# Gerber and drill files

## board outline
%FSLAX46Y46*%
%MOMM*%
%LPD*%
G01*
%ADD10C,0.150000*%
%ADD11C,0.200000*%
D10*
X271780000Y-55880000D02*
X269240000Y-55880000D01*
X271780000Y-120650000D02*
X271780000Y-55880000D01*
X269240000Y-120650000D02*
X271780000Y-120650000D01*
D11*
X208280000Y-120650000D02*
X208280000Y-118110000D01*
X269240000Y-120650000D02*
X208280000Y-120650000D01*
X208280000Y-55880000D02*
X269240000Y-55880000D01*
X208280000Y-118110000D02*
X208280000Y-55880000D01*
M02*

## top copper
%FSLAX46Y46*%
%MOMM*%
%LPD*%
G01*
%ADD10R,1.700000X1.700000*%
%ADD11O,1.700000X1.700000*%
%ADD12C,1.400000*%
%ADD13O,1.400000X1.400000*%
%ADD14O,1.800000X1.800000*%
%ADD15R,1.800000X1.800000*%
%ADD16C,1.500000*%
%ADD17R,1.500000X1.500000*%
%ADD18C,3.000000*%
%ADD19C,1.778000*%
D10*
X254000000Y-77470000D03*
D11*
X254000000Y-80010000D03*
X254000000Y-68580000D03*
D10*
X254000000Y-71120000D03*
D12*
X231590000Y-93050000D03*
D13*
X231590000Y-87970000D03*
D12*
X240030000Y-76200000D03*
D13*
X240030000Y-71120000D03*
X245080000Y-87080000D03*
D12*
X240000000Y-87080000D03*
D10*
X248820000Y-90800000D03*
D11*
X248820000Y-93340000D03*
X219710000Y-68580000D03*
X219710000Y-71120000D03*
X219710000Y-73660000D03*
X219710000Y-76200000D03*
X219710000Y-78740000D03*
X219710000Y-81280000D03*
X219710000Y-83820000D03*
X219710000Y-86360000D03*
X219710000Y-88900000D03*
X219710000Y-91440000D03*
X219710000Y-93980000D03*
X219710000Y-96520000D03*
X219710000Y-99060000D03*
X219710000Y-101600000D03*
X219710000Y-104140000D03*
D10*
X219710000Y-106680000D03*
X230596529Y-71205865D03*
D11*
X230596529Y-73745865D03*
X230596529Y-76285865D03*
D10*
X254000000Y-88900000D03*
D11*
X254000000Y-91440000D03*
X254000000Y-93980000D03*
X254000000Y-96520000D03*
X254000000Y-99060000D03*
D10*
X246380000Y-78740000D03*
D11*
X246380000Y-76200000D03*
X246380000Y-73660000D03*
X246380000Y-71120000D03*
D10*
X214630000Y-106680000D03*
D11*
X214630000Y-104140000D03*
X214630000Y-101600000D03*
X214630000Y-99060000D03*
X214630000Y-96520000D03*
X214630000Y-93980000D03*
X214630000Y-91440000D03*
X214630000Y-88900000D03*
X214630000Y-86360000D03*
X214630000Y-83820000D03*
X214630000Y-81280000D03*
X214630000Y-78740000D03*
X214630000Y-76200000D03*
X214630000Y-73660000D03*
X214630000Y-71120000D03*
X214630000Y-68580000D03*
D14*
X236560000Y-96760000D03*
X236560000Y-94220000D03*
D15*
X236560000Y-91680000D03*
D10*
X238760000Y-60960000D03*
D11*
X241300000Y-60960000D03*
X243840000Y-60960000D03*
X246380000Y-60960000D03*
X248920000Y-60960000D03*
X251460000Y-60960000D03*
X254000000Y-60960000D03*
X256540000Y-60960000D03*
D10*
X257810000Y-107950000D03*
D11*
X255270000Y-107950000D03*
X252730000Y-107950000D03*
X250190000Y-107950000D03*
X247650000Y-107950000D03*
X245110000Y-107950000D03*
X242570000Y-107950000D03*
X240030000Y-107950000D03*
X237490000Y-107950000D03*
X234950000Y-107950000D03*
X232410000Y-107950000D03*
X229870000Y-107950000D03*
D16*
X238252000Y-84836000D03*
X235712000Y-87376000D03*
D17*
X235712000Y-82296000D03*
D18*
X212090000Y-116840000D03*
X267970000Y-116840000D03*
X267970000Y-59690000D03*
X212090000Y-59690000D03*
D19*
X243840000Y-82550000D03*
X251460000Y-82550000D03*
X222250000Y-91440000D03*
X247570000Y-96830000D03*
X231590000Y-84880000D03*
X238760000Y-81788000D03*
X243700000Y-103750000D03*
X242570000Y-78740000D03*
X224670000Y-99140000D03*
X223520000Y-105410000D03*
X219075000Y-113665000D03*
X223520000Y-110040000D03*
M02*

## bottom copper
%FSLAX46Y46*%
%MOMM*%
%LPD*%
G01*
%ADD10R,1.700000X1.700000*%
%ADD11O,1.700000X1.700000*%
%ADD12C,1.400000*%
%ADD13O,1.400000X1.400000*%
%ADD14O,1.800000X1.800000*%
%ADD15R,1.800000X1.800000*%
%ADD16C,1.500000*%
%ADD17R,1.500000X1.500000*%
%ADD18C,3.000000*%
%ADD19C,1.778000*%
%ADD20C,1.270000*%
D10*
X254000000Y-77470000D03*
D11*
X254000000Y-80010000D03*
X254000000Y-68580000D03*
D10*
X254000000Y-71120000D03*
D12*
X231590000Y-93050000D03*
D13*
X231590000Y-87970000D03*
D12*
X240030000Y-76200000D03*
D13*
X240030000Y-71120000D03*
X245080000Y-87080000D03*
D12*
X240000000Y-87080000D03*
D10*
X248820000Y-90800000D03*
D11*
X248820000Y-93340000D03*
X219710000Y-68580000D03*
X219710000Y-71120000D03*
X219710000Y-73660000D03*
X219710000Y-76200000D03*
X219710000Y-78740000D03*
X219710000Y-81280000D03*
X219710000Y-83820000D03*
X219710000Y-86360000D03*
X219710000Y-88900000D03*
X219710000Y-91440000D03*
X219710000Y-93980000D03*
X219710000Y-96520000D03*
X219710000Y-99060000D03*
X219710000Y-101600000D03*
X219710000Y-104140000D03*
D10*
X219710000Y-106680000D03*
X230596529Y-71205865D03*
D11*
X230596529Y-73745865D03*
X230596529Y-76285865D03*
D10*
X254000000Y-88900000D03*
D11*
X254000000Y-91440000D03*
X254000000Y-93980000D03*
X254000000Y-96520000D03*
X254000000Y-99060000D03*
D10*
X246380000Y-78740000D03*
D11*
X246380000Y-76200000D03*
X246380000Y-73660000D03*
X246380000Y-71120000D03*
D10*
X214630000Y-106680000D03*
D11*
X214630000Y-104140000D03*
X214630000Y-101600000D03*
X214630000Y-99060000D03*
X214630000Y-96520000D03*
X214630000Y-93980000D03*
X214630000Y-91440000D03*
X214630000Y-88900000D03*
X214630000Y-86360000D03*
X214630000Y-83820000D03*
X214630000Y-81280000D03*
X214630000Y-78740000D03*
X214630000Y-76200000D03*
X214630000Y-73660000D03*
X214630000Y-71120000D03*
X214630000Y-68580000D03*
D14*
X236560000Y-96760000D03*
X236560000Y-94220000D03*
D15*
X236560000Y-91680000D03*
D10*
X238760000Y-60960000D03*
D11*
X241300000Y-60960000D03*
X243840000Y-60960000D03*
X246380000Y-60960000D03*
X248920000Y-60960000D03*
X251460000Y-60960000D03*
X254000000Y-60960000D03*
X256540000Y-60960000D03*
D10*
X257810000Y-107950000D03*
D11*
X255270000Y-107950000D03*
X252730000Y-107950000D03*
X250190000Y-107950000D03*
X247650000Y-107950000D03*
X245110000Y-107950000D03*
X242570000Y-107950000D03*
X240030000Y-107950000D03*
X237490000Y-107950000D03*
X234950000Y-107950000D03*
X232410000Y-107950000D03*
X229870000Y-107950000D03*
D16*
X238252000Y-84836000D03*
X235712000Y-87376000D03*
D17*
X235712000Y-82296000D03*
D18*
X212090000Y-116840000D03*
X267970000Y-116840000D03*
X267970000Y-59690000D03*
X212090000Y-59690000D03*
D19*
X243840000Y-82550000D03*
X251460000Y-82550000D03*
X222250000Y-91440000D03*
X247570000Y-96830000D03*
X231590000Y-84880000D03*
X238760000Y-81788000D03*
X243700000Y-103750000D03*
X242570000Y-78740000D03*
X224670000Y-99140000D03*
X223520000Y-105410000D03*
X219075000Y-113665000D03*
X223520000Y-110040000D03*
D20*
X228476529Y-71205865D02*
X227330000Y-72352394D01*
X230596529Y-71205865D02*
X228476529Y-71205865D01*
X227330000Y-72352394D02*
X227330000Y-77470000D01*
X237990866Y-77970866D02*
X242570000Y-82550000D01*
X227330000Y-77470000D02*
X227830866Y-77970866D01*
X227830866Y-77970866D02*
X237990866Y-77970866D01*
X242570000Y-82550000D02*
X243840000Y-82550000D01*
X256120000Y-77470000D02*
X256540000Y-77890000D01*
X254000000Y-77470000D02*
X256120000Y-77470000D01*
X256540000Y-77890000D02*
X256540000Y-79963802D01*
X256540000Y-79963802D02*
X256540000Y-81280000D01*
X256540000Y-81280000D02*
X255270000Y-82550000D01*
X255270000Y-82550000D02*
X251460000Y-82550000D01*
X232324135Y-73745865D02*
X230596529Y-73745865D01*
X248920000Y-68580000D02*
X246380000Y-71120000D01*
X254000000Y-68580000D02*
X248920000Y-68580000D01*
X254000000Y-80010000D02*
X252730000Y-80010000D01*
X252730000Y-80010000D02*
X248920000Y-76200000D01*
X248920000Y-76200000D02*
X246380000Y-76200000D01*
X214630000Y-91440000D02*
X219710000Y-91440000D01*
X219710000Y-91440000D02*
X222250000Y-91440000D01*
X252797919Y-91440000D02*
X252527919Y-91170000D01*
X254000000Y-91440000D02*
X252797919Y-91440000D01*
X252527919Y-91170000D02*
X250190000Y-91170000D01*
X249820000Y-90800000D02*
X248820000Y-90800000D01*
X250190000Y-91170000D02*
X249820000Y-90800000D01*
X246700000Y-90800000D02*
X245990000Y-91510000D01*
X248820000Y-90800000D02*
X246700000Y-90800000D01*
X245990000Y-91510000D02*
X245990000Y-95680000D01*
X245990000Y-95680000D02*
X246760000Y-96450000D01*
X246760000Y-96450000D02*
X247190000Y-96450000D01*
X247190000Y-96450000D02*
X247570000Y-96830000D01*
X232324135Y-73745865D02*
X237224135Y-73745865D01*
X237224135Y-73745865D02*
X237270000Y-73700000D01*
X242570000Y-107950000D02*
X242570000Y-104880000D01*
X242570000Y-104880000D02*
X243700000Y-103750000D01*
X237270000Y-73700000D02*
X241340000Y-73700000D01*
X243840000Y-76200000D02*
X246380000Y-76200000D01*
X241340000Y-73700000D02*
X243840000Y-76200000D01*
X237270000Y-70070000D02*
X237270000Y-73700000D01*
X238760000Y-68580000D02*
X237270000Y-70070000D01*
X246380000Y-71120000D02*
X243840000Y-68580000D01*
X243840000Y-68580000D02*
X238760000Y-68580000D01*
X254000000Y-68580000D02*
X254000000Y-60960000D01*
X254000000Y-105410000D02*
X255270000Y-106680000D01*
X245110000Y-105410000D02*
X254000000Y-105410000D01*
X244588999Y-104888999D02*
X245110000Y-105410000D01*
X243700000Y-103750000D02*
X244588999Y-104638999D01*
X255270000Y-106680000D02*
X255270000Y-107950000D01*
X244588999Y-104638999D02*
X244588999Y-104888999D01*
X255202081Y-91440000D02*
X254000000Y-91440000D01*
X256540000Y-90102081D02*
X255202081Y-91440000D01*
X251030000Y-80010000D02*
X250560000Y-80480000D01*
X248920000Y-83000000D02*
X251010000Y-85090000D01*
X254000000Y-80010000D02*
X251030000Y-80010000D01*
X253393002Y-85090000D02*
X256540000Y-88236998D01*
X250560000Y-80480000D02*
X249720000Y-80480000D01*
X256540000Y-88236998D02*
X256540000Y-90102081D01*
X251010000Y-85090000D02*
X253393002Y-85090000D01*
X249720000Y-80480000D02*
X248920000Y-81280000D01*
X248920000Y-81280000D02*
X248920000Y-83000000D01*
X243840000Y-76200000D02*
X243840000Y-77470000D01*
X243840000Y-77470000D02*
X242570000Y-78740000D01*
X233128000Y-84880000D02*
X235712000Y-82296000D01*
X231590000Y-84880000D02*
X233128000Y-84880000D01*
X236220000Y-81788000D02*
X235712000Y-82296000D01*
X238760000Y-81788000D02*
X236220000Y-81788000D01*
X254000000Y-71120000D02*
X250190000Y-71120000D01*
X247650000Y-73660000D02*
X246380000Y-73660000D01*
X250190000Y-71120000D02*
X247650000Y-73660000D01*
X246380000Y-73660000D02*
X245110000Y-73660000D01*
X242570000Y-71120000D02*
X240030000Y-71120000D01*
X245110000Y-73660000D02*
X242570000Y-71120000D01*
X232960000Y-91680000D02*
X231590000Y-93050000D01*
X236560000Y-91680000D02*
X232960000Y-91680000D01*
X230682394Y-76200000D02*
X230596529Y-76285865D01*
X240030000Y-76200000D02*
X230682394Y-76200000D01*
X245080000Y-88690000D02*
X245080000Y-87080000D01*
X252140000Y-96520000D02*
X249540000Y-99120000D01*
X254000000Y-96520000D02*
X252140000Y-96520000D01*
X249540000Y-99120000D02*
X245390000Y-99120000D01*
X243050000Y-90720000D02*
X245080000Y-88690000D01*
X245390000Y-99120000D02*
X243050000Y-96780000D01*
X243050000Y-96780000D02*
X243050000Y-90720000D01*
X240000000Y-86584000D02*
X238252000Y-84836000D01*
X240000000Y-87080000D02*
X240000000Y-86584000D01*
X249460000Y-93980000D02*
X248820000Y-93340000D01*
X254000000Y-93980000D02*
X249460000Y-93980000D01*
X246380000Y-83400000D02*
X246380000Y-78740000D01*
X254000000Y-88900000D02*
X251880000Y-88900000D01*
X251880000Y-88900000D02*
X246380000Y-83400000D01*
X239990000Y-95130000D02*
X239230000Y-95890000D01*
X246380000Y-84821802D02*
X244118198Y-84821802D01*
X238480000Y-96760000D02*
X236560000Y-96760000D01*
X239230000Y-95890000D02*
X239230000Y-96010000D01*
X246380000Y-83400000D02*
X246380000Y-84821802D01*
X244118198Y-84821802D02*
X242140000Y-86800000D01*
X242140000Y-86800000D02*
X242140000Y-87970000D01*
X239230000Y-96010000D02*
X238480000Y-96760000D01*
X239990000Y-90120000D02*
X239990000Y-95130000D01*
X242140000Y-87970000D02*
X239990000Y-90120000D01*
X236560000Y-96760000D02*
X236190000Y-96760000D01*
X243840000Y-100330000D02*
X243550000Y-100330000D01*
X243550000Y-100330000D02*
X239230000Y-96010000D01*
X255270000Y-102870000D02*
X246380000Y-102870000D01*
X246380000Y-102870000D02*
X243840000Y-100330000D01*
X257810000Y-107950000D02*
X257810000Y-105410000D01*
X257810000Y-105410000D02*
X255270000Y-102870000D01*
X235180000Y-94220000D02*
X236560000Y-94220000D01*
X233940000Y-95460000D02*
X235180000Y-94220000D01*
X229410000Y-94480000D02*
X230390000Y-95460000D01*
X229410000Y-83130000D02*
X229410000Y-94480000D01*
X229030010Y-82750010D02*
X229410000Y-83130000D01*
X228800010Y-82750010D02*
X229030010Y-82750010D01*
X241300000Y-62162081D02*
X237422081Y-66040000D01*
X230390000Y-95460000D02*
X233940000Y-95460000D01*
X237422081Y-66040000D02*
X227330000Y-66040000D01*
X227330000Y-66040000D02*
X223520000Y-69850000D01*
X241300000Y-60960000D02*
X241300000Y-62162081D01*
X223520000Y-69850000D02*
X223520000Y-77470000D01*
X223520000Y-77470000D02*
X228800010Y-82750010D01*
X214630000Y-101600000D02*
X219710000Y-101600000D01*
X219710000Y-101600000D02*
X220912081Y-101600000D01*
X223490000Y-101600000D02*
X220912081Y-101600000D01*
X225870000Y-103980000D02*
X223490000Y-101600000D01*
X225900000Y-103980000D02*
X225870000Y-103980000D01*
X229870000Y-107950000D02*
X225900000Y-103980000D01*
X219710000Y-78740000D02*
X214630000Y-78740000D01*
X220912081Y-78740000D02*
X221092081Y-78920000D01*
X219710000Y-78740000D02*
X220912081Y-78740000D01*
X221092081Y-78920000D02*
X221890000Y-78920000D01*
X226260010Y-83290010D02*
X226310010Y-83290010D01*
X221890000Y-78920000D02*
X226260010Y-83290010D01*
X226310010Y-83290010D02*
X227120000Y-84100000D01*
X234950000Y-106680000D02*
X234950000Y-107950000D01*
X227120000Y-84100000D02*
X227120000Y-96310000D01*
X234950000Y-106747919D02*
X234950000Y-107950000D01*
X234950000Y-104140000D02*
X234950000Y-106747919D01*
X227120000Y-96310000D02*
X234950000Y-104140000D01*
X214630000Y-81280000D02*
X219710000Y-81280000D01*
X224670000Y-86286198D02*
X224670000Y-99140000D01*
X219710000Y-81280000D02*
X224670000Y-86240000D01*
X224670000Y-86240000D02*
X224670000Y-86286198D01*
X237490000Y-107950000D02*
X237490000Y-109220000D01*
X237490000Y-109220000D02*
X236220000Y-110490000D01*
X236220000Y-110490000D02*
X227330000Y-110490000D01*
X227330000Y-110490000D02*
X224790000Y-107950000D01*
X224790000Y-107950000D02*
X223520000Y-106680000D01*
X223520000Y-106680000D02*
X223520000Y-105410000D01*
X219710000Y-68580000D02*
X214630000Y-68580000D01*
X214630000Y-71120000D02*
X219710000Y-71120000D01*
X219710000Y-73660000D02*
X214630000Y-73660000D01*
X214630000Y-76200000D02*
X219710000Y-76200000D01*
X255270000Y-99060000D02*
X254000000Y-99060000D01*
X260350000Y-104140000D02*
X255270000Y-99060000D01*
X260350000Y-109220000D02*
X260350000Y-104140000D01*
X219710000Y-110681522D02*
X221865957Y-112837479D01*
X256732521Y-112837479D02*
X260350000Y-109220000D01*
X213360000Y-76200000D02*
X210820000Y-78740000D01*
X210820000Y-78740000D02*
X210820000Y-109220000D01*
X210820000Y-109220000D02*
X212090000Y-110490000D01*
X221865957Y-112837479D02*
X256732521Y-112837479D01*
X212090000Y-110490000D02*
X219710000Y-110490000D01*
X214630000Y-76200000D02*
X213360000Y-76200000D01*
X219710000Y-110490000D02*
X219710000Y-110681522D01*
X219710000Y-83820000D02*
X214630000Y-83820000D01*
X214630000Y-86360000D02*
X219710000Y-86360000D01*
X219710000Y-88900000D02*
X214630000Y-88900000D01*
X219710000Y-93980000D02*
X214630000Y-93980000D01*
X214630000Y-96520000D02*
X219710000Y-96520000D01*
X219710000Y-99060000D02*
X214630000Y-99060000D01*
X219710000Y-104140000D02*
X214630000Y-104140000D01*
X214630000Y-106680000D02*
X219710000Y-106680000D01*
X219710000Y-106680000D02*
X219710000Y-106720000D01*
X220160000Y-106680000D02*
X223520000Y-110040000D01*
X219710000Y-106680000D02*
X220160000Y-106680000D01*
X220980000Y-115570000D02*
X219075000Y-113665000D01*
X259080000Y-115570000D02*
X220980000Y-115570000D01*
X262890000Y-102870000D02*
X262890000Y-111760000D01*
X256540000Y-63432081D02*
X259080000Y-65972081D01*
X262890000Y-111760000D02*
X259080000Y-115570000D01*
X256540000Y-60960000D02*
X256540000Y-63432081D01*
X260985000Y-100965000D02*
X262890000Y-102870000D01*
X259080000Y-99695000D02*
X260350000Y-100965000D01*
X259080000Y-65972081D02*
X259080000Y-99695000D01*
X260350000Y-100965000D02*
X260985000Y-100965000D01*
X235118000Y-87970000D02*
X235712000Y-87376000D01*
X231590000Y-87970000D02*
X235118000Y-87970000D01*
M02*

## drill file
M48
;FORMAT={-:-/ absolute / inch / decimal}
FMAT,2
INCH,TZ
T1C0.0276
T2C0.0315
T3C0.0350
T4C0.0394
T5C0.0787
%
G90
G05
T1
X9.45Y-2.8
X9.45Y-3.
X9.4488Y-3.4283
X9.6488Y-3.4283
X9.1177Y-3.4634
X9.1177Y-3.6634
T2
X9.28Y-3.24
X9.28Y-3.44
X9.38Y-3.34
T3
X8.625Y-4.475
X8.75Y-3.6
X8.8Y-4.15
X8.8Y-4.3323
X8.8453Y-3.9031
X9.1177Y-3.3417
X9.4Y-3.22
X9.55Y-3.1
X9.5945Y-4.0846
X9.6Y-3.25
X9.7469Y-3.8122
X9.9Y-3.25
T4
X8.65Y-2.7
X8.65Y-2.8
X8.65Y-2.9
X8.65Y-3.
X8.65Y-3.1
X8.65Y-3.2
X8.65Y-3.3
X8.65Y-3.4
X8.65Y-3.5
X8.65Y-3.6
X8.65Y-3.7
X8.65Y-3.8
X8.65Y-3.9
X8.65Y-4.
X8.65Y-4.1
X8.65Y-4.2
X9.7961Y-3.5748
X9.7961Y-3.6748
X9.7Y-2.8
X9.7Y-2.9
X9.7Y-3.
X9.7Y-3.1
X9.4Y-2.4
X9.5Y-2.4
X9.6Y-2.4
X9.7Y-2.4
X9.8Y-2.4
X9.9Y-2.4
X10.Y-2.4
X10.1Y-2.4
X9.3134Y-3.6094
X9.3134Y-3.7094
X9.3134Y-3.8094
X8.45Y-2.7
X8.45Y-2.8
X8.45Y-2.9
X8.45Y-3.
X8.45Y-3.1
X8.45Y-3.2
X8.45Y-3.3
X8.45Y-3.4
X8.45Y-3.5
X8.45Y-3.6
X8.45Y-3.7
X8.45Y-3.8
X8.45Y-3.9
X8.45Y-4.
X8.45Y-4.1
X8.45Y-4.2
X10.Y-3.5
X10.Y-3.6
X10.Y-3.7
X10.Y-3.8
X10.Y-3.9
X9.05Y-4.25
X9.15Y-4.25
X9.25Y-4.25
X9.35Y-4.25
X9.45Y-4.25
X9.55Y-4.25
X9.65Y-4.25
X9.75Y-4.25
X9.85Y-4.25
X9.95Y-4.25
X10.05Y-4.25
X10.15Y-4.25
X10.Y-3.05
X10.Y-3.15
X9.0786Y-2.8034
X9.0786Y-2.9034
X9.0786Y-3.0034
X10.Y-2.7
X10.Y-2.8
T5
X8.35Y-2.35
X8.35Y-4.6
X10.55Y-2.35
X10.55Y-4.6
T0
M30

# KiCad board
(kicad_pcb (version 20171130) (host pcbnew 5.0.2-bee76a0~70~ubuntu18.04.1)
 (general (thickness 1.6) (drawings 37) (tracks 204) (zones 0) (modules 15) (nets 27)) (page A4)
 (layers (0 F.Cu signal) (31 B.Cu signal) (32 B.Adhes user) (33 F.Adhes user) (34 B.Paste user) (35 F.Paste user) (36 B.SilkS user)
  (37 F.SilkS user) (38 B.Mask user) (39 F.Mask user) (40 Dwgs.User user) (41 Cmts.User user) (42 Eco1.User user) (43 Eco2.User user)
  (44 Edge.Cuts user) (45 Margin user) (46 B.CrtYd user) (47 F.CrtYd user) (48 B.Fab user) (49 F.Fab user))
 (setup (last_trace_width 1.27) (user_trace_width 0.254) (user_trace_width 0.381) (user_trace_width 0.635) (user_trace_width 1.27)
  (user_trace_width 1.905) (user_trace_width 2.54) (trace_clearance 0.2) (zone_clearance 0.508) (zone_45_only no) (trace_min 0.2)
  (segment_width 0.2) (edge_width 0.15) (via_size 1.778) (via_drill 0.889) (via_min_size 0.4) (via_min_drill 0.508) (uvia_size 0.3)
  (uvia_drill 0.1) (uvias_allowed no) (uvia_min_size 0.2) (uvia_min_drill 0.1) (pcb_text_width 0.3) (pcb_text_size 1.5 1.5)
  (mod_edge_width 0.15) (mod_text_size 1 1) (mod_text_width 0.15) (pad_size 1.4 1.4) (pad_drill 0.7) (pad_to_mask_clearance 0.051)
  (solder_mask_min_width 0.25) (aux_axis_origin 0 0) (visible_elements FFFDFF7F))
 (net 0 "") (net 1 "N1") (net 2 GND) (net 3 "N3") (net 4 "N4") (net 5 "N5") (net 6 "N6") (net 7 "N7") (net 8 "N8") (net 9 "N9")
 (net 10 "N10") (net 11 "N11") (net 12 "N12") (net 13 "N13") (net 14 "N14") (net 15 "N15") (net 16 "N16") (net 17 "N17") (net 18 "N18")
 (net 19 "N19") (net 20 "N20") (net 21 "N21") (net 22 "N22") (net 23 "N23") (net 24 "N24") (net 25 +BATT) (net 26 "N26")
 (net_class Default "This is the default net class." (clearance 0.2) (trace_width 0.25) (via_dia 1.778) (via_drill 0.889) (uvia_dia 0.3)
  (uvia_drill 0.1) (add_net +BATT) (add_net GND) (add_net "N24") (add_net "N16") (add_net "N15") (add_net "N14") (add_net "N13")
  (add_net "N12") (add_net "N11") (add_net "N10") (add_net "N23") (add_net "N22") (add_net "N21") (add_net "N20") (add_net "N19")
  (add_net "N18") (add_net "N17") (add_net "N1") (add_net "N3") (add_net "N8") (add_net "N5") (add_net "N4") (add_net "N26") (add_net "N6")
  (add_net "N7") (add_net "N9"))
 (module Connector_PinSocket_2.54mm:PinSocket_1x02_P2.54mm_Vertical (layer F.Cu) (at 254 77.47)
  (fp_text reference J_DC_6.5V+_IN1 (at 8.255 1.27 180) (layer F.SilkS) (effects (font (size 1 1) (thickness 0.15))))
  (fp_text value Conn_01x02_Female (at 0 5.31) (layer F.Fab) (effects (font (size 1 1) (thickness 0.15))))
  (pad 1 thru_hole rect (at 0 0) (size 1.7 1.7) (drill 1) (layers *.Cu *.Mask) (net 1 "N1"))
  (pad 2 thru_hole oval (at 0 2.54) (size 1.7 1.7) (drill 1) (layers *.Cu *.Mask) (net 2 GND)))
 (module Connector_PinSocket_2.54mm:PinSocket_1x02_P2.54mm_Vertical (layer F.Cu) (at 254 71.12 180)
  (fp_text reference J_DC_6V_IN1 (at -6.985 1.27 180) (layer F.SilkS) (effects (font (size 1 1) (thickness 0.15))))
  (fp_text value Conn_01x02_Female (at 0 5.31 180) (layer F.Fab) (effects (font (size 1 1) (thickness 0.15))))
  (pad 2 thru_hole oval (at 0 2.54 180) (size 1.7 1.7) (drill 1) (layers *.Cu *.Mask) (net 2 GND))
  (pad 1 thru_hole rect (at 0 0 180) (size 1.7 1.7) (drill 1) (layers *.Cu *.Mask) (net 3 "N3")))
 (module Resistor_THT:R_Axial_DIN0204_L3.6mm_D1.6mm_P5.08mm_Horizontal (layer F.Cu) (at 231.59 93.05 90)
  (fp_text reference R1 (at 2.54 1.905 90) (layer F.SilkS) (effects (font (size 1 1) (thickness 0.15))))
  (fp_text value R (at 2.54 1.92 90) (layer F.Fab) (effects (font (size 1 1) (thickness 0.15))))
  (pad 1 thru_hole circle (at 0 0 90) (size 1.4 1.4) (drill 0.7) (layers *.Cu *.Mask) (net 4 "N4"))
  (pad 2 thru_hole oval (at 5.08 0 90) (size 1.4 1.4) (drill 0.7) (layers *.Cu *.Mask) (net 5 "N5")))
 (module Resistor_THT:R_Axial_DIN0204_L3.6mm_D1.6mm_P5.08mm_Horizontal (layer F.Cu) (at 240.03 76.2 90)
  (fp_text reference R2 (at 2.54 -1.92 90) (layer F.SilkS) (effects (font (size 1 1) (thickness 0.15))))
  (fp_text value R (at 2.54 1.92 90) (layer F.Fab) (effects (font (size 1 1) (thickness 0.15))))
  (pad 1 thru_hole circle (at 0 0 90) (size 1.4 1.4) (drill 0.7) (layers *.Cu *.Mask) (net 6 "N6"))
  (pad 2 thru_hole oval (at 5.08 0 90) (size 1.4 1.4) (drill 0.7) (layers *.Cu *.Mask) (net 3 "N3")))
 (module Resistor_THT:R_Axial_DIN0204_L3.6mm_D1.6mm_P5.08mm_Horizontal (layer F.Cu) (at 240 87.08)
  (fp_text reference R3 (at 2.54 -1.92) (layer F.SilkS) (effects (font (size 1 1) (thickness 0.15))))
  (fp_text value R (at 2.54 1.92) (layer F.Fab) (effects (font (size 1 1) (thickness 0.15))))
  (pad 2 thru_hole oval (at 5.08 0) (size 1.4 1.4) (drill 0.7) (layers *.Cu *.Mask) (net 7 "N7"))
  (pad 1 thru_hole circle (at 0 0) (size 1.4 1.4) (drill 0.7) (layers *.Cu *.Mask) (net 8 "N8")))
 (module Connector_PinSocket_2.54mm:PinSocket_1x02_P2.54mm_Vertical (layer F.Cu) (at 248.82 90.8)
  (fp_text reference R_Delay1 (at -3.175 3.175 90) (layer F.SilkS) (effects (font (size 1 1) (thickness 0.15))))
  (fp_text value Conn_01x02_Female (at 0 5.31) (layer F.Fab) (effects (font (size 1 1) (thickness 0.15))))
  (pad 1 thru_hole rect (at 0 0) (size 1.7 1.7) (drill 1) (layers *.Cu *.Mask) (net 2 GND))
  (pad 2 thru_hole oval (at 0 2.54) (size 1.7 1.7) (drill 1) (layers *.Cu *.Mask) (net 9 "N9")))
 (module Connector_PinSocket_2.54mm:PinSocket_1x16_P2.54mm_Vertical (layer F.Cu) (at 219.71 106.68 180)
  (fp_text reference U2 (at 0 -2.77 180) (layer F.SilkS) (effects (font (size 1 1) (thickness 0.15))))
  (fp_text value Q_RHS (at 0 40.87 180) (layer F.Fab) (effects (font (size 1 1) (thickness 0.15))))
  (pad 16 thru_hole oval (at 0 38.1 180) (size 1.7 1.7) (drill 1) (layers *.Cu *.Mask) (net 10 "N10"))
  (pad 15 thru_hole oval (at 0 35.56 180) (size 1.7 1.7) (drill 1) (layers *.Cu *.Mask) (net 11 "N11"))
  (pad 14 thru_hole oval (at 0 33.02 180) (size 1.7 1.7) (drill 1) (layers *.Cu *.Mask) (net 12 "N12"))
  (pad 13 thru_hole oval (at 0 30.48 180) (size 1.7 1.7) (drill 1) (layers *.Cu *.Mask) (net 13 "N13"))
  (pad 12 thru_hole oval (at 0 27.94 180) (size 1.7 1.7) (drill 1) (layers *.Cu *.Mask) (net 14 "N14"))
  (pad 11 thru_hole oval (at 0 25.4 180) (size 1.7 1.7) (drill 1) (layers *.Cu *.Mask) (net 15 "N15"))
  (pad 10 thru_hole oval (at 0 22.86 180) (size 1.7 1.7) (drill 1) (layers *.Cu *.Mask) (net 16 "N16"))
  (pad 9 thru_hole oval (at 0 20.32 180) (size 1.7 1.7) (drill 1) (layers *.Cu *.Mask) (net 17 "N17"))
  (pad 8 thru_hole oval (at 0 17.78 180) (size 1.7 1.7) (drill 1) (layers *.Cu *.Mask) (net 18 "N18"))
  (pad 7 thru_hole oval (at 0 15.24 180) (size 1.7 1.7) (drill 1) (layers *.Cu *.Mask) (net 2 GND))
  (pad 6 thru_hole oval (at 0 12.7 180) (size 1.7 1.7) (drill 1) (layers *.Cu *.Mask) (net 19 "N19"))
  (pad 5 thru_hole oval (at 0 10.16 180) (size 1.7 1.7) (drill 1) (layers *.Cu *.Mask) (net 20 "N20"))
  (pad 4 thru_hole oval (at 0 7.62 180) (size 1.7 1.7) (drill 1) (layers *.Cu *.Mask) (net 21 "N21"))
  (pad 3 thru_hole oval (at 0 5.08 180) (size 1.7 1.7) (drill 1) (layers *.Cu *.Mask) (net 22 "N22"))
  (pad 2 thru_hole oval (at 0 2.54 180) (size 1.7 1.7) (drill 1) (layers *.Cu *.Mask) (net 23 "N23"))
  (pad 1 thru_hole rect (at 0 0 180) (size 1.7 1.7) (drill 1) (layers *.Cu *.Mask) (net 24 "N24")))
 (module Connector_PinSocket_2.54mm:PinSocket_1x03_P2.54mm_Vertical (layer F.Cu) (at 230.596529 71.205865)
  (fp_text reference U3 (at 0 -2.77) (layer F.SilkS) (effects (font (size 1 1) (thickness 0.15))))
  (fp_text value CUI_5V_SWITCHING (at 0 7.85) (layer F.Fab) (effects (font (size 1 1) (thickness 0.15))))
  (pad 1 thru_hole rect (at 0 0) (size 1.7 1.7) (drill 1) (layers *.Cu *.Mask) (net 1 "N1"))
  (pad 2 thru_hole oval (at 0 2.54) (size 1.7 1.7) (drill 1) (layers *.Cu *.Mask) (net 2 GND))
  (pad 3 thru_hole oval (at 0 5.08) (size 1.7 1.7) (drill 1) (layers *.Cu *.Mask) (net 6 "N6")))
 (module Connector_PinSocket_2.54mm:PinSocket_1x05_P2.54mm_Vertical (layer F.Cu) (at 254 88.9)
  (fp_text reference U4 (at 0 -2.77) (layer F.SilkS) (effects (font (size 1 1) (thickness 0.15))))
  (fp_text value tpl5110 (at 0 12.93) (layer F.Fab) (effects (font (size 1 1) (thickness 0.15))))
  (pad 1 thru_hole rect (at 0 0) (size 1.7 1.7) (drill 1) (layers *.Cu *.Mask) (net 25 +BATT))
  (pad 2 thru_hole oval (at 0 2.54) (size 1.7 1.7) (drill 1) (layers *.Cu *.Mask) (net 2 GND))
  (pad 3 thru_hole oval (at 0 5.08) (size 1.7 1.7) (drill 1) (layers *.Cu *.Mask) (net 9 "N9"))
  (pad 4 thru_hole oval (at 0 7.62) (size 1.7 1.7) (drill 1) (layers *.Cu *.Mask) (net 7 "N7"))
  (pad 5 thru_hole oval (at 0 10.16) (size 1.7 1.7) (drill 1) (layers *.Cu *.Mask) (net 13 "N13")))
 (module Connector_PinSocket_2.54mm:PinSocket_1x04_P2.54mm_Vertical (layer F.Cu) (at 246.38 78.74 180)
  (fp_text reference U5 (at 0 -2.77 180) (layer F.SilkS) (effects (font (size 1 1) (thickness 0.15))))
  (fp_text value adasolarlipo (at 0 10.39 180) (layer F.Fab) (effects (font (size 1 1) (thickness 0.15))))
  (pad 1 thru_hole rect (at 0 0 180) (size 1.7 1.7) (drill 1) (layers *.Cu *.Mask) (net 25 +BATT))
  (pad 2 thru_hole oval (at 0 2.54 180) (size 1.7 1.7) (drill 1) (layers *.Cu *.Mask) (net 2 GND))
  (pad 3 thru_hole oval (at 0 5.08 180) (size 1.7 1.7) (drill 1) (layers *.Cu *.Mask) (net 3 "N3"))
  (pad 4 thru_hole oval (at 0 7.62 180) (size 1.7 1.7) (drill 1) (layers *.Cu *.Mask) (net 2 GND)))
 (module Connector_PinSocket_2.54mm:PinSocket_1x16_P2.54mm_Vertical (layer F.Cu) (at 214.63 106.68 180)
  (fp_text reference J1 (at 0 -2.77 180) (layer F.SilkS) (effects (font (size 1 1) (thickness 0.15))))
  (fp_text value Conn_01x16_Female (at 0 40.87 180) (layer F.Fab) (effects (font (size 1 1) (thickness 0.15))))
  (pad 1 thru_hole rect (at 0 0 180) (size 1.7 1.7) (drill 1) (layers *.Cu *.Mask) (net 24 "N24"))
  (pad 2 thru_hole oval (at 0 2.54 180) (size 1.7 1.7) (drill 1) (layers *.Cu *.Mask) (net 23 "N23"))
  (pad 3 thru_hole oval (at 0 5.08 180) (size 1.7 1.7) (drill 1) (layers *.Cu *.Mask) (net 22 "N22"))
  (pad 4 thru_hole oval (at 0 7.62 180) (size 1.7 1.7) (drill 1) (layers *.Cu *.Mask) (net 21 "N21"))
  (pad 5 thru_hole oval (at 0 10.16 180) (size 1.7 1.7) (drill 1) (layers *.Cu *.Mask) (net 20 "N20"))
  (pad 6 thru_hole oval (at 0 12.7 180) (size 1.7 1.7) (drill 1) (layers *.Cu *.Mask) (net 19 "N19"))
  (pad 7 thru_hole oval (at 0 15.24 180) (size 1.7 1.7) (drill 1) (layers *.Cu *.Mask) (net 2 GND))
  (pad 8 thru_hole oval (at 0 17.78 180) (size 1.7 1.7) (drill 1) (layers *.Cu *.Mask) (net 18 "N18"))
  (pad 9 thru_hole oval (at 0 20.32 180) (size 1.7 1.7) (drill 1) (layers *.Cu *.Mask) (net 17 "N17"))
  (pad 10 thru_hole oval (at 0 22.86 180) (size 1.7 1.7) (drill 1) (layers *.Cu *.Mask) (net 16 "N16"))
  (pad 11 thru_hole oval (at 0 25.4 180) (size 1.7 1.7) (drill 1) (layers *.Cu *.Mask) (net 15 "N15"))
  (pad 12 thru_hole oval (at 0 27.94 180) (size 1.7 1.7) (drill 1) (layers *.Cu *.Mask) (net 14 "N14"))
  (pad 13 thru_hole oval (at 0 30.48 180) (size 1.7 1.7) (drill 1) (layers *.Cu *.Mask) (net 13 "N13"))
  (pad 14 thru_hole oval (at 0 33.02 180) (size 1.7 1.7) (drill 1) (layers *.Cu *.Mask) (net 12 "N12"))
  (pad 15 thru_hole oval (at 0 35.56 180) (size 1.7 1.7) (drill 1) (layers *.Cu *.Mask) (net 11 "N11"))
  (pad 16 thru_hole oval (at 0 38.1 180) (size 1.7 1.7) (drill 1) (layers *.Cu *.Mask) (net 10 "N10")))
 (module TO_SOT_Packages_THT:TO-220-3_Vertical (layer F.Cu) (at 236.56 91.68 270)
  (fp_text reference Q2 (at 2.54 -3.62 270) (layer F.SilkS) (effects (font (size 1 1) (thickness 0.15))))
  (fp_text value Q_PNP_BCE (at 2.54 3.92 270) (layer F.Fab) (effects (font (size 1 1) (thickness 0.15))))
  (pad 3 thru_hole oval (at 5.08 0 270) (size 1.8 1.8) (drill 1) (layers *.Cu *.Mask) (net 25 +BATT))
  (pad 2 thru_hole oval (at 2.54 0 270) (size 1.8 1.8) (drill 1) (layers *.Cu *.Mask) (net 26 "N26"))
  (pad 1 thru_hole rect (at 0 0 270) (size 1.8 1.8) (drill 1) (layers *.Cu *.Mask) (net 4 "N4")))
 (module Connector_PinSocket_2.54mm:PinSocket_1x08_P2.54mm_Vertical (layer F.Cu) (at 238.76 60.96 90)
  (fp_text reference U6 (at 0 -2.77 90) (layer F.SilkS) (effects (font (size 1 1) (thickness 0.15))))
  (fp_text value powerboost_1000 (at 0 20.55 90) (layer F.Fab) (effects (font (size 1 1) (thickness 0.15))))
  (pad 1 thru_hole rect (at 0 0 90) (size 1.7 1.7) (drill 1) (layers *.Cu *.Mask))
  (pad 2 thru_hole oval (at 0 2.54 90) (size 1.7 1.7) (drill 1) (layers *.Cu *.Mask) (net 26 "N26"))
  (pad 3 thru_hole oval (at 0 5.08 90) (size 1.7 1.7) (drill 1) (layers *.Cu *.Mask))
  (pad 4 thru_hole oval (at 0 7.62 90) (size 1.7 1.7) (drill 1) (layers *.Cu *.Mask))
  (pad 5 thru_hole oval (at 0 10.16 90) (size 1.7 1.7) (drill 1) (layers *.Cu *.Mask))
  (pad 6 thru_hole oval (at 0 12.7 90) (size 1.7 1.7) (drill 1) (layers *.Cu *.Mask))
  (pad 7 thru_hole oval (at 0 15.24 90) (size 1.7 1.7) (drill 1) (layers *.Cu *.Mask) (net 2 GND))
  (pad 8 thru_hole oval (at 0 17.78 90) (size 1.7 1.7) (drill 1) (layers *.Cu *.Mask) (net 24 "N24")))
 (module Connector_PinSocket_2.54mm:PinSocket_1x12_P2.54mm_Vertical (layer F.Cu) (at 257.81 107.95 270)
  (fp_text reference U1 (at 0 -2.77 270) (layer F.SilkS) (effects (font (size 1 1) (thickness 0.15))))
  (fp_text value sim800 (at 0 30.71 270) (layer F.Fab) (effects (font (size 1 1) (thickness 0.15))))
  (pad 1 thru_hole rect (at 0 0 270) (size 1.7 1.7) (drill 1) (layers *.Cu *.Mask) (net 25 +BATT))
  (pad 2 thru_hole oval (at 0 2.54 270) (size 1.7 1.7) (drill 1) (layers *.Cu *.Mask) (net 2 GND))
  (pad 3 thru_hole oval (at 0 5.08 270) (size 1.7 1.7) (drill 1) (layers *.Cu *.Mask))
  (pad 4 thru_hole oval (at 0 7.62 270) (size 1.7 1.7) (drill 1) (layers *.Cu *.Mask))
  (pad 5 thru_hole oval (at 0 10.16 270) (size 1.7 1.7) (drill 1) (layers *.Cu *.Mask))
  (pad 6 thru_hole oval (at 0 12.7 270) (size 1.7 1.7) (drill 1) (layers *.Cu *.Mask))
  (pad 7 thru_hole oval (at 0 15.24 270) (size 1.7 1.7) (drill 1) (layers *.Cu *.Mask) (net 2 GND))
  (pad 8 thru_hole oval (at 0 17.78 270) (size 1.7 1.7) (drill 1) (layers *.Cu *.Mask))
  (pad 9 thru_hole oval (at 0 20.32 270) (size 1.7 1.7) (drill 1) (layers *.Cu *.Mask) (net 15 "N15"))
  (pad 10 thru_hole oval (at 0 22.86 270) (size 1.7 1.7) (drill 1) (layers *.Cu *.Mask) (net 14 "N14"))
  (pad 11 thru_hole oval (at 0 25.4 270) (size 1.7 1.7) (drill 1) (layers *.Cu *.Mask))
  (pad 12 thru_hole oval (at 0 27.94 270) (size 1.7 1.7) (drill 1) (layers *.Cu *.Mask) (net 22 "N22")))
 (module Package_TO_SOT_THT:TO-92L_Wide (layer F.Cu) (at 235.712 82.296 270)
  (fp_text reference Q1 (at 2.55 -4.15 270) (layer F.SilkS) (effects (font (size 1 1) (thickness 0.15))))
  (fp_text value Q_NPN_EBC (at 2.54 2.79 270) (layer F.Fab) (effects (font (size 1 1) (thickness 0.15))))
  (pad 2 thru_hole circle (at 2.54 -2.54) (size 1.5 1.5) (drill 0.8) (layers *.Cu *.Mask) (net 8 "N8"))
  (pad 3 thru_hole circle (at 5.08 0) (size 1.5 1.5) (drill 0.8) (layers *.Cu *.Mask) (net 5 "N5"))
  (pad 1 thru_hole rect (at 0 0) (size 1.5 1.5) (drill 0.8) (layers *.Cu *.Mask) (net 2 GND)))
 (gr_line (start 271.78 55.88) (end 269.24 55.88) (layer Edge.Cuts) (width 0.15))
 (gr_line (start 271.78 120.65) (end 271.78 55.88) (layer Edge.Cuts) (width 0.15))
 (gr_line (start 269.24 120.65) (end 271.78 120.65) (layer Edge.Cuts) (width 0.15))
 (gr_line (start 208.28 120.65) (end 208.28 118.11) (layer Edge.Cuts) (width 0.2))
 (gr_line (start 269.24 120.65) (end 208.28 120.65) (layer Edge.Cuts) (width 0.2))
 (gr_line (start 208.28 55.88) (end 269.24 55.88) (layer Edge.Cuts) (width 0.2))
 (gr_line (start 208.28 118.11) (end 208.28 55.88) (layer Edge.Cuts) (width 0.2))
 (via (at 212.09 116.84) (size 3) (drill 2) (layers F.Cu B.Cu) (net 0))
 (via (at 267.97 116.84) (size 3) (drill 2) (layers F.Cu B.Cu) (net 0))
 (via (at 267.97 59.69) (size 3) (drill 2) (layers F.Cu B.Cu) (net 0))
 (via (at 212.09 59.69) (size 3) (drill 2) (layers F.Cu B.Cu) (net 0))
 (segment (start 228.476529 71.205865) (end 227.33 72.352394) (width 1.27) (layer B.Cu) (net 1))
 (segment (start 230.596529 71.205865) (end 228.476529 71.205865) (width 1.27) (layer B.Cu) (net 1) (status 10))
 (segment (start 227.33 72.352394) (end 227.33 77.47) (width 1.27) (layer B.Cu) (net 1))
 (segment (start 237.990866 77.970866) (end 242.57 82.55) (width 1.27) (layer B.Cu) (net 1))
 (segment (start 227.33 77.47) (end 227.830866 77.970866) (width 1.27) (layer B.Cu) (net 1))
 (segment (start 227.830866 77.970866) (end 237.990866 77.970866) (width 1.27) (layer B.Cu) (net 1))
 (via (at 243.84 82.55) (size 1.778) (drill 0.889) (layers F.Cu B.Cu) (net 1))
 (segment (start 242.57 82.55) (end 243.84 82.55) (width 1.27) (layer B.Cu) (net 1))
 (segment (start 256.12 77.47) (end 256.54 77.89) (width 1.27) (layer B.Cu) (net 1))
 (segment (start 254 77.47) (end 256.12 77.47) (width 1.27) (layer B.Cu) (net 1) (status 10))
 (segment (start 256.54 77.89) (end 256.54 79.963802) (width 1.27) (layer B.Cu) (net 1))
 (segment (start 256.54 79.963802) (end 256.54 81.28) (width 1.27) (layer B.Cu) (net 1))
 (segment (start 256.54 81.28) (end 255.27 82.55) (width 1.27) (layer B.Cu) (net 1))
 (via (at 251.46 82.55) (size 1.778) (drill 0.889) (layers F.Cu B.Cu) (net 1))
 (segment (start 255.27 82.55) (end 251.46 82.55) (width 1.27) (layer B.Cu) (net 1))
 (segment (start 232.324135 73.745865) (end 230.596529 73.745865) (width 1.27) (layer B.Cu) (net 2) (status 20))
 (segment (start 248.92 68.58) (end 246.38 71.12) (width 1.27) (layer B.Cu) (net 2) (status 20))
 (segment (start 254 68.58) (end 248.92 68.58) (width 1.27) (layer B.Cu) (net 2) (status 10))
 (segment (start 254 80.01) (end 252.73 80.01) (width 1.27) (layer B.Cu) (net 2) (status 10))
 (segment (start 252.73 80.01) (end 248.92 76.2) (width 1.27) (layer B.Cu) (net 2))
 (segment (start 248.92 76.2) (end 246.38 76.2) (width 1.27) (layer B.Cu) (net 2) (status 20))
 (segment (start 214.63 91.44) (end 219.71 91.44) (width 1.27) (layer B.Cu) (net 2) (status 30))
 (via (at 222.25 91.44) (size 1.778) (drill 0.889) (layers F.Cu B.Cu) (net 2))
 (segment (start 219.71 91.44) (end 222.25 91.44) (width 1.27) (layer B.Cu) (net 2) (status 10))
 (segment (start 252.797919 91.44) (end 252.527919 91.17) (width 1.27) (layer B.Cu) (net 2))
 (segment (start 254 91.44) (end 252.797919 91.44) (width 1.27) (layer B.Cu) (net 2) (status 10))
 (segment (start 252.527919 91.17) (end 250.19 91.17) (width 1.27) (layer B.Cu) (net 2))
 (segment (start 249.82 90.8) (end 248.82 90.8) (width 1.27) (layer B.Cu) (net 2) (status 20))
 (segment (start 250.19 91.17) (end 249.82 90.8) (width 1.27) (layer B.Cu) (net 2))
 (segment (start 246.7 90.8) (end 245.99 91.51) (width 1.27) (layer B.Cu) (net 2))
 (segment (start 248.82 90.8) (end 246.7 90.8) (width 1.27) (layer B.Cu) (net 2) (status 10))
 (segment (start 245.99 91.51) (end 245.99 95.68) (width 1.27) (layer B.Cu) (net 2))
 (segment (start 245.99 95.68) (end 246.76 96.45) (width 1.27) (layer B.Cu) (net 2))
 (via (at 247.57 96.83) (size 1.778) (drill 0.889) (layers F.Cu B.Cu) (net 2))
 (segment (start 246.76 96.45) (end 247.19 96.45) (width 1.27) (layer B.Cu) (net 2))
 (segment (start 247.19 96.45) (end 247.57 96.83) (width 1.27) (layer B.Cu) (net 2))
 (via (at 231.59 84.88) (size 1.778) (drill 0.889) (layers F.Cu B.Cu) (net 2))
 (via (at 238.76 81.788) (size 1.778) (drill 0.889) (layers F.Cu B.Cu) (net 2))
 (segment (start 232.324135 73.745865) (end 237.224135 73.745865) (width 1.27) (layer B.Cu) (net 2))
 (segment (start 237.224135 73.745865) (end 237.27 73.7) (width 1.27) (layer B.Cu) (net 2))
 (segment (start 254 71.12) (end 250.19 71.12) (width 1.27) (layer B.Cu) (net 3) (status 10))
 (segment (start 247.65 73.66) (end 246.38 73.66) (width 1.27) (layer B.Cu) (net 3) (status 20))
 (segment (start 250.19 71.12) (end 247.65 73.66) (width 1.27) (layer B.Cu) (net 3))
 (segment (start 232.96 91.68) (end 231.59 93.05) (width 1.27) (layer B.Cu) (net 4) (status 20))
 (segment (start 236.56 91.68) (end 232.96 91.68) (width 1.27) (layer B.Cu) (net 4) (status 10))
 (segment (start 230.682394 76.2) (end 230.596529 76.285865) (width 1.27) (layer B.Cu) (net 6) (status 30))
 (segment (start 240.03 76.2) (end 230.682394 76.2) (width 1.27) (layer B.Cu) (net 6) (status 30))
 (segment (start 245.08 88.69) (end 245.08 87.08) (width 1.27) (layer B.Cu) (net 7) (status 20))
 (segment (start 252.14 96.52) (end 249.54 99.12) (width 1.27) (layer B.Cu) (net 7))
 (segment (start 254 96.52) (end 252.14 96.52) (width 1.27) (layer B.Cu) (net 7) (status 10))
 (segment (start 249.54 99.12) (end 245.39 99.12) (width 1.27) (layer B.Cu) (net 7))
 (segment (start 243.05 90.72) (end 245.08 88.69) (width 1.27) (layer B.Cu) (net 7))
 (segment (start 245.39 99.12) (end 243.05 96.78) (width 1.27) (layer B.Cu) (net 7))
 (segment (start 243.05 96.78) (end 243.05 90.72) (width 1.27) (layer B.Cu) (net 7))
 (segment (start 249.46 93.98) (end 248.82 93.34) (width 1.27) (layer B.Cu) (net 9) (status 30))
 (segment (start 254 93.98) (end 249.46 93.98) (width 1.27) (layer B.Cu) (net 9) (status 30))
 (segment (start 246.38 83.4) (end 246.38 78.74) (width 1.27) (layer B.Cu) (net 25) (status 20))
 (segment (start 254 88.9) (end 251.88 88.9) (width 1.27) (layer B.Cu) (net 25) (status 10))
 (segment (start 251.88 88.9) (end 246.38 83.4) (width 1.27) (layer B.Cu) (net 25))
 (segment (start 239.99 95.13) (end 239.23 95.89) (width 1.27) (layer B.Cu) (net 25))
 (segment (start 246.38 84.821802) (end 244.118198 84.821802) (width 1.27) (layer B.Cu) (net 25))
 (segment (start 238.48 96.76) (end 236.56 96.76) (width 1.27) (layer B.Cu) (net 25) (status 20))
 (segment (start 239.23 95.89) (end 239.23 96.01) (width 1.27) (layer B.Cu) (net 25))
 (segment (start 246.38 83.4) (end 246.38 84.821802) (width 1.27) (layer B.Cu) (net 25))
 (segment (start 244.118198 84.821802) (end 242.14 86.8) (width 1.27) (layer B.Cu) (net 25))
 (segment (start 242.14 86.8) (end 242.14 87.97) (width 1.27) (layer B.Cu) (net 25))
 (segment (start 239.23 96.01) (end 238.48 96.76) (width 1.27) (layer B.Cu) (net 25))
 (segment (start 239.99 90.12) (end 239.99 95.13) (width 1.27) (layer B.Cu) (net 25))
 (segment (start 242.14 87.97) (end 239.99 90.12) (width 1.27) (layer B.Cu) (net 25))
 (segment (start 236.56 96.76) (end 236.19 96.76) (width 1.27) (layer B.Cu) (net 25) (status 30))
 (segment (start 214.63 101.6) (end 219.71 101.6) (width 1.27) (layer B.Cu) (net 22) (status 30))
 (segment (start 219.71 101.6) (end 220.912081 101.6) (width 1.27) (layer B.Cu) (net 22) (status 10))
 (segment (start 223.49 101.6) (end 220.912081 101.6) (width 1.27) (layer B.Cu) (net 22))
 (segment (start 225.87 103.98) (end 223.49 101.6) (width 1.27) (layer B.Cu) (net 22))
 (segment (start 219.71 78.74) (end 214.63 78.74) (width 1.27) (layer B.Cu) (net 14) (status 30))
 (via (at 243.7 103.75) (size 1.778) (drill 0.889) (layers F.Cu B.Cu) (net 2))
 (segment (start 242.57 107.95) (end 242.57 104.88) (width 1.27) (layer B.Cu) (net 2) (status 10))
 (segment (start 242.57 104.88) (end 243.7 103.75) (width 1.27) (layer B.Cu) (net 2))
 (segment (start 220.912081 78.74) (end 221.092081 78.92) (width 1.27) (layer B.Cu) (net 14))
 (segment (start 219.71 78.74) (end 220.912081 78.74) (width 1.27) (layer B.Cu) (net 14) (status 10))
 (segment (start 221.092081 78.92) (end 221.89 78.92) (width 1.27) (layer B.Cu) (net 14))
 (segment (start 226.26001 83.29001) (end 226.31001 83.29001) (width 1.27) (layer B.Cu) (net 14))
 (segment (start 221.89 78.92) (end 226.26001 83.29001) (width 1.27) (layer B.Cu) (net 14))
 (segment (start 226.31001 83.29001) (end 227.12 84.1) (width 1.27) (layer B.Cu) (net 14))
 (segment (start 214.63 81.28) (end 219.71 81.28) (width 1.27) (layer B.Cu) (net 15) (status 30))
 (segment (start 237.27 73.7) (end 241.34 73.7) (width 1.27) (layer B.Cu) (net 2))
 (segment (start 243.84 76.2) (end 246.38 76.2) (width 1.27) (layer B.Cu) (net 2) (status 20))
 (segment (start 241.34 73.7) (end 243.84 76.2) (width 1.27) (layer B.Cu) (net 2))
 (segment (start 237.27 70.07) (end 237.27 73.7) (width 1.27) (layer B.Cu) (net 2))
 (segment (start 238.76 68.58) (end 237.27 70.07) (width 1.27) (layer B.Cu) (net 2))
 (segment (start 246.38 71.12) (end 243.84 68.58) (width 1.27) (layer B.Cu) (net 2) (status 10))
 (segment (start 243.84 68.58) (end 238.76 68.58) (width 1.27) (layer B.Cu) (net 2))
 (segment (start 254 68.58) (end 254 60.96) (width 1.27) (layer B.Cu) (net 2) (status 30))
 (segment (start 254 105.41) (end 255.27 106.68) (width 1.27) (layer B.Cu) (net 2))
 (segment (start 245.11 105.41) (end 254 105.41) (width 1.27) (layer B.Cu) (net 2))
 (segment (start 244.588999 104.888999) (end 245.11 105.41) (width 1.27) (layer B.Cu) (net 2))
 (segment (start 243.7 103.75) (end 244.588999 104.638999) (width 1.27) (layer B.Cu) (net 2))
 (segment (start 255.27 106.68) (end 255.27 107.95) (width 1.27) (layer B.Cu) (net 2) (status 20))
 (segment (start 244.588999 104.638999) (end 244.588999 104.888999) (width 1.27) (layer B.Cu) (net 2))
 (segment (start 255.202081 91.44) (end 254 91.44) (width 1.27) (layer B.Cu) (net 2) (status 20))
 (segment (start 256.54 90.102081) (end 255.202081 91.44) (width 1.27) (layer B.Cu) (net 2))
 (segment (start 251.03 80.01) (end 250.56 80.48) (width 1.27) (layer B.Cu) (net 2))
 (segment (start 248.92 83) (end 251.01 85.09) (width 1.27) (layer B.Cu) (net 2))
 (segment (start 254 80.01) (end 251.03 80.01) (width 1.27) (layer B.Cu) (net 2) (status 10))
 (segment (start 253.393002 85.09) (end 256.54 88.236998) (width 1.27) (layer B.Cu) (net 2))
 (segment (start 250.56 80.48) (end 249.72 80.48) (width 1.27) (layer B.Cu) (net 2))
 (segment (start 256.54 88.236998) (end 256.54 90.102081) (width 1.27) (layer B.Cu) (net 2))
 (segment (start 251.01 85.09) (end 253.393002 85.09) (width 1.27) (layer B.Cu) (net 2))
 (segment (start 249.72 80.48) (end 248.92 81.28) (width 1.27) (layer B.Cu) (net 2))
 (segment (start 248.92 81.28) (end 248.92 83) (width 1.27) (layer B.Cu) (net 2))
 (via (at 242.57 78.74) (size 1.778) (drill 0.889) (layers F.Cu B.Cu) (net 2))
 (segment (start 243.84 76.2) (end 243.84 77.47) (width 1.27) (layer B.Cu) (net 2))
 (segment (start 243.84 77.47) (end 242.57 78.74) (width 1.27) (layer B.Cu) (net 2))
 (segment (start 233.128 84.88) (end 235.712 82.296) (width 1.27) (layer B.Cu) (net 2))
 (segment (start 231.59 84.88) (end 233.128 84.88) (width 1.27) (layer B.Cu) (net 2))
 (segment (start 236.22 81.788) (end 235.712 82.296) (width 1.27) (layer B.Cu) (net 2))
 (segment (start 238.76 81.788) (end 236.22 81.788) (width 1.27) (layer B.Cu) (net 2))
 (segment (start 246.38 73.66) (end 245.11 73.66) (width 1.27) (layer B.Cu) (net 3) (status 10))
 (segment (start 242.57 71.12) (end 240.03 71.12) (width 1.27) (layer B.Cu) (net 3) (status 20))
 (segment (start 245.11 73.66) (end 242.57 71.12) (width 1.27) (layer B.Cu) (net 3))
 (segment (start 240 86.584) (end 238.252 84.836) (width 1.27) (layer B.Cu) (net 8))
 (segment (start 240 87.08) (end 240 86.584) (width 1.27) (layer B.Cu) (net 8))
 (segment (start 243.84 100.33) (end 243.55 100.33) (width 1.27) (layer B.Cu) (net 25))
 (segment (start 243.55 100.33) (end 239.23 96.01) (width 1.27) (layer B.Cu) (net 25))
 (segment (start 255.27 102.87) (end 246.38 102.87) (width 1.27) (layer B.Cu) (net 25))
 (segment (start 246.38 102.87) (end 243.84 100.33) (width 1.27) (layer B.Cu) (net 25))
 (segment (start 257.81 107.95) (end 257.81 105.41) (width 1.27) (layer B.Cu) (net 25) (status 10))
 (segment (start 257.81 105.41) (end 255.27 102.87) (width 1.27) (layer B.Cu) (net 25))
 (segment (start 235.18 94.22) (end 236.56 94.22) (width 1.27) (layer B.Cu) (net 26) (status 20))
 (segment (start 233.94 95.46) (end 235.18 94.22) (width 1.27) (layer B.Cu) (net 26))
 (segment (start 229.41 94.48) (end 230.39 95.46) (width 1.27) (layer B.Cu) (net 26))
 (segment (start 229.41 83.13) (end 229.41 94.48) (width 1.27) (layer B.Cu) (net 26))
 (segment (start 229.03001 82.75001) (end 229.41 83.13) (width 1.27) (layer B.Cu) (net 26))
 (segment (start 228.80001 82.75001) (end 229.03001 82.75001) (width 1.27) (layer B.Cu) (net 26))
 (segment (start 241.3 62.162081) (end 237.422081 66.04) (width 1.27) (layer B.Cu) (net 26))
 (segment (start 230.39 95.46) (end 233.94 95.46) (width 1.27) (layer B.Cu) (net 26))
 (segment (start 237.422081 66.04) (end 227.33 66.04) (width 1.27) (layer B.Cu) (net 26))
 (segment (start 227.33 66.04) (end 223.52 69.85) (width 1.27) (layer B.Cu) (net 26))
 (segment (start 241.3 60.96) (end 241.3 62.162081) (width 1.27) (layer B.Cu) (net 26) (status 10))
 (segment (start 223.52 69.85) (end 223.52 77.47) (width 1.27) (layer B.Cu) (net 26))
 (segment (start 223.52 77.47) (end 228.80001 82.75001) (width 1.27) (layer B.Cu) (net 26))
 (segment (start 225.9 103.98) (end 225.87 103.98) (width 1.27) (layer B.Cu) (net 22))
 (segment (start 229.87 107.95) (end 225.9 103.98) (width 1.27) (layer B.Cu) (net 22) (status 10))
 (segment (start 234.95 106.68) (end 234.95 107.95) (width 1.27) (layer B.Cu) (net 14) (status 20))
 (segment (start 227.12 84.1) (end 227.12 96.31) (width 1.27) (layer B.Cu) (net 14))
 (segment (start 234.95 106.747919) (end 234.95 107.95) (width 1.27) (layer B.Cu) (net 14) (status 20))
 (segment (start 234.95 104.14) (end 234.95 106.747919) (width 1.27) (layer B.Cu) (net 14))
 (segment (start 227.12 96.31) (end 234.95 104.14) (width 1.27) (layer B.Cu) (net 14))
 (via (at 224.67 99.14) (size 1.778) (drill 0.889) (layers F.Cu B.Cu) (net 15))
 (segment (start 224.67 86.286198) (end 224.67 99.14) (width 1.27) (layer B.Cu) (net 15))
 (segment (start 219.71 81.28) (end 224.67 86.24) (width 1.27) (layer B.Cu) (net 15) (status 10))
 (segment (start 224.67 86.24) (end 224.67 86.286198) (width 1.27) (layer B.Cu) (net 15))
 (segment (start 237.49 107.95) (end 237.49 109.22) (width 1.27) (layer B.Cu) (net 15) (status 10))
 (segment (start 237.49 109.22) (end 236.22 110.49) (width 1.27) (layer B.Cu) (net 15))
 (segment (start 236.22 110.49) (end 227.33 110.49) (width 1.27) (layer B.Cu) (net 15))
 (segment (start 227.33 110.49) (end 224.79 107.95) (width 1.27) (layer B.Cu) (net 15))
 (segment (start 224.79 107.95) (end 223.52 106.68) (width 1.27) (layer B.Cu) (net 15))
 (via (at 223.52 105.41) (size 1.778) (drill 0.889) (layers F.Cu B.Cu) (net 15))
 (segment (start 223.52 106.68) (end 223.52 105.41) (width 1.27) (layer B.Cu) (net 15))
 (segment (start 219.71 68.58) (end 214.63 68.58) (width 1.27) (layer B.Cu) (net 10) (status 30))
 (segment (start 214.63 71.12) (end 219.71 71.12) (width 1.27) (layer B.Cu) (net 11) (status 30))
 (segment (start 219.71 73.66) (end 214.63 73.66) (width 1.27) (layer B.Cu) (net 12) (status 30))
 (segment (start 214.63 76.2) (end 219.71 76.2) (width 1.27) (layer B.Cu) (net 13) (status 30))
 (segment (start 255.27 99.06) (end 254 99.06) (width 1.27) (layer B.Cu) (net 13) (status 20))
 (segment (start 260.35 104.14) (end 255.27 99.06) (width 1.27) (layer B.Cu) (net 13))
 (segment (start 260.35 109.22) (end 260.35 104.14) (width 1.27) (layer B.Cu) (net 13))
 (segment (start 219.71 110.681522) (end 221.865957 112.837479) (width 1.27) (layer B.Cu) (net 13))
 (segment (start 256.732521 112.837479) (end 260.35 109.22) (width 1.27) (layer B.Cu) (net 13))
 (segment (start 213.36 76.2) (end 210.82 78.74) (width 1.27) (layer B.Cu) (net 13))
 (segment (start 210.82 78.74) (end 210.82 109.22) (width 1.27) (layer B.Cu) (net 13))
 (segment (start 210.82 109.22) (end 212.09 110.49) (width 1.27) (layer B.Cu) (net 13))
 (segment (start 221.865957 112.837479) (end 256.732521 112.837479) (width 1.27) (layer B.Cu) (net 13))
 (segment (start 212.09 110.49) (end 219.71 110.49) (width 1.27) (layer B.Cu) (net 13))
 (segment (start 214.63 76.2) (end 213.36 76.2) (width 1.27) (layer B.Cu) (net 13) (status 10))
 (segment (start 219.71 110.49) (end 219.71 110.681522) (width 1.27) (layer B.Cu) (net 13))
 (segment (start 219.71 83.82) (end 214.63 83.82) (width 1.27) (layer B.Cu) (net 16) (status 30))
 (segment (start 214.63 86.36) (end 219.71 86.36) (width 1.27) (layer B.Cu) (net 17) (status 30))
 (segment (start 219.71 88.9) (end 214.63 88.9) (width 1.27) (layer B.Cu) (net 18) (status 30))
 (segment (start 219.71 93.98) (end 214.63 93.98) (width 1.27) (layer B.Cu) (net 19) (status 30))
 (segment (start 214.63 96.52) (end 219.71 96.52) (width 1.27) (layer B.Cu) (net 20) (status 30))
 (segment (start 219.71 99.06) (end 214.63 99.06) (width 1.27) (layer B.Cu) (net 21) (status 30))
 (segment (start 219.71 104.14) (end 214.63 104.14) (width 1.27) (layer B.Cu) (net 23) (status 30))
 (segment (start 214.63 106.68) (end 219.71 106.68) (width 1.27) (layer B.Cu) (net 24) (status 30))
 (via (at 219.075 113.665) (size 1.778) (drill 0.889) (layers F.Cu B.Cu) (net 24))
 (segment (start 219.71 106.68) (end 219.71 106.72) (width 1.27) (layer B.Cu) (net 24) (status 30))
 (via (at 223.52 110.04) (size 1.778) (drill 0.889) (layers F.Cu B.Cu) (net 24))
 (segment (start 220.16 106.68) (end 223.52 110.04) (width 1.27) (layer B.Cu) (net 24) (status 10))
 (segment (start 219.71 106.68) (end 220.16 106.68) (width 1.27) (layer B.Cu) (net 24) (status 30))
 (segment (start 220.98 115.57) (end 219.075 113.665) (width 1.27) (layer B.Cu) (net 24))
 (segment (start 259.08 115.57) (end 220.98 115.57) (width 1.27) (layer B.Cu) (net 24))
 (segment (start 262.89 102.87) (end 262.89 111.76) (width 1.27) (layer B.Cu) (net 24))
 (segment (start 256.54 63.432081) (end 259.08 65.972081) (width 1.27) (layer B.Cu) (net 24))
 (segment (start 259.08 65.972081) (end 259.08 99.695) (width 1.27) (layer B.Cu) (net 24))
 (segment (start 262.89 111.76) (end 259.08 115.57) (width 1.27) (layer B.Cu) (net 24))
 (segment (start 259.08 99.695) (end 260.35 100.965) (width 1.27) (layer B.Cu) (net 24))
 (segment (start 256.54 60.96) (end 256.54 63.432081) (width 1.27) (layer B.Cu) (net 24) (status 10))
 (segment (start 260.35 100.965) (end 260.985 100.965) (width 1.27) (layer B.Cu) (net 24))
 (segment (start 260.985 100.965) (end 262.89 102.87) (width 1.27) (layer B.Cu) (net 24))
 (segment (start 235.118 87.97) (end 235.712 87.376) (width 1.27) (layer B.Cu) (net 5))
 (segment (start 231.59 87.97) (end 235.118 87.97) (width 1.27) (layer B.Cu) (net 5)))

